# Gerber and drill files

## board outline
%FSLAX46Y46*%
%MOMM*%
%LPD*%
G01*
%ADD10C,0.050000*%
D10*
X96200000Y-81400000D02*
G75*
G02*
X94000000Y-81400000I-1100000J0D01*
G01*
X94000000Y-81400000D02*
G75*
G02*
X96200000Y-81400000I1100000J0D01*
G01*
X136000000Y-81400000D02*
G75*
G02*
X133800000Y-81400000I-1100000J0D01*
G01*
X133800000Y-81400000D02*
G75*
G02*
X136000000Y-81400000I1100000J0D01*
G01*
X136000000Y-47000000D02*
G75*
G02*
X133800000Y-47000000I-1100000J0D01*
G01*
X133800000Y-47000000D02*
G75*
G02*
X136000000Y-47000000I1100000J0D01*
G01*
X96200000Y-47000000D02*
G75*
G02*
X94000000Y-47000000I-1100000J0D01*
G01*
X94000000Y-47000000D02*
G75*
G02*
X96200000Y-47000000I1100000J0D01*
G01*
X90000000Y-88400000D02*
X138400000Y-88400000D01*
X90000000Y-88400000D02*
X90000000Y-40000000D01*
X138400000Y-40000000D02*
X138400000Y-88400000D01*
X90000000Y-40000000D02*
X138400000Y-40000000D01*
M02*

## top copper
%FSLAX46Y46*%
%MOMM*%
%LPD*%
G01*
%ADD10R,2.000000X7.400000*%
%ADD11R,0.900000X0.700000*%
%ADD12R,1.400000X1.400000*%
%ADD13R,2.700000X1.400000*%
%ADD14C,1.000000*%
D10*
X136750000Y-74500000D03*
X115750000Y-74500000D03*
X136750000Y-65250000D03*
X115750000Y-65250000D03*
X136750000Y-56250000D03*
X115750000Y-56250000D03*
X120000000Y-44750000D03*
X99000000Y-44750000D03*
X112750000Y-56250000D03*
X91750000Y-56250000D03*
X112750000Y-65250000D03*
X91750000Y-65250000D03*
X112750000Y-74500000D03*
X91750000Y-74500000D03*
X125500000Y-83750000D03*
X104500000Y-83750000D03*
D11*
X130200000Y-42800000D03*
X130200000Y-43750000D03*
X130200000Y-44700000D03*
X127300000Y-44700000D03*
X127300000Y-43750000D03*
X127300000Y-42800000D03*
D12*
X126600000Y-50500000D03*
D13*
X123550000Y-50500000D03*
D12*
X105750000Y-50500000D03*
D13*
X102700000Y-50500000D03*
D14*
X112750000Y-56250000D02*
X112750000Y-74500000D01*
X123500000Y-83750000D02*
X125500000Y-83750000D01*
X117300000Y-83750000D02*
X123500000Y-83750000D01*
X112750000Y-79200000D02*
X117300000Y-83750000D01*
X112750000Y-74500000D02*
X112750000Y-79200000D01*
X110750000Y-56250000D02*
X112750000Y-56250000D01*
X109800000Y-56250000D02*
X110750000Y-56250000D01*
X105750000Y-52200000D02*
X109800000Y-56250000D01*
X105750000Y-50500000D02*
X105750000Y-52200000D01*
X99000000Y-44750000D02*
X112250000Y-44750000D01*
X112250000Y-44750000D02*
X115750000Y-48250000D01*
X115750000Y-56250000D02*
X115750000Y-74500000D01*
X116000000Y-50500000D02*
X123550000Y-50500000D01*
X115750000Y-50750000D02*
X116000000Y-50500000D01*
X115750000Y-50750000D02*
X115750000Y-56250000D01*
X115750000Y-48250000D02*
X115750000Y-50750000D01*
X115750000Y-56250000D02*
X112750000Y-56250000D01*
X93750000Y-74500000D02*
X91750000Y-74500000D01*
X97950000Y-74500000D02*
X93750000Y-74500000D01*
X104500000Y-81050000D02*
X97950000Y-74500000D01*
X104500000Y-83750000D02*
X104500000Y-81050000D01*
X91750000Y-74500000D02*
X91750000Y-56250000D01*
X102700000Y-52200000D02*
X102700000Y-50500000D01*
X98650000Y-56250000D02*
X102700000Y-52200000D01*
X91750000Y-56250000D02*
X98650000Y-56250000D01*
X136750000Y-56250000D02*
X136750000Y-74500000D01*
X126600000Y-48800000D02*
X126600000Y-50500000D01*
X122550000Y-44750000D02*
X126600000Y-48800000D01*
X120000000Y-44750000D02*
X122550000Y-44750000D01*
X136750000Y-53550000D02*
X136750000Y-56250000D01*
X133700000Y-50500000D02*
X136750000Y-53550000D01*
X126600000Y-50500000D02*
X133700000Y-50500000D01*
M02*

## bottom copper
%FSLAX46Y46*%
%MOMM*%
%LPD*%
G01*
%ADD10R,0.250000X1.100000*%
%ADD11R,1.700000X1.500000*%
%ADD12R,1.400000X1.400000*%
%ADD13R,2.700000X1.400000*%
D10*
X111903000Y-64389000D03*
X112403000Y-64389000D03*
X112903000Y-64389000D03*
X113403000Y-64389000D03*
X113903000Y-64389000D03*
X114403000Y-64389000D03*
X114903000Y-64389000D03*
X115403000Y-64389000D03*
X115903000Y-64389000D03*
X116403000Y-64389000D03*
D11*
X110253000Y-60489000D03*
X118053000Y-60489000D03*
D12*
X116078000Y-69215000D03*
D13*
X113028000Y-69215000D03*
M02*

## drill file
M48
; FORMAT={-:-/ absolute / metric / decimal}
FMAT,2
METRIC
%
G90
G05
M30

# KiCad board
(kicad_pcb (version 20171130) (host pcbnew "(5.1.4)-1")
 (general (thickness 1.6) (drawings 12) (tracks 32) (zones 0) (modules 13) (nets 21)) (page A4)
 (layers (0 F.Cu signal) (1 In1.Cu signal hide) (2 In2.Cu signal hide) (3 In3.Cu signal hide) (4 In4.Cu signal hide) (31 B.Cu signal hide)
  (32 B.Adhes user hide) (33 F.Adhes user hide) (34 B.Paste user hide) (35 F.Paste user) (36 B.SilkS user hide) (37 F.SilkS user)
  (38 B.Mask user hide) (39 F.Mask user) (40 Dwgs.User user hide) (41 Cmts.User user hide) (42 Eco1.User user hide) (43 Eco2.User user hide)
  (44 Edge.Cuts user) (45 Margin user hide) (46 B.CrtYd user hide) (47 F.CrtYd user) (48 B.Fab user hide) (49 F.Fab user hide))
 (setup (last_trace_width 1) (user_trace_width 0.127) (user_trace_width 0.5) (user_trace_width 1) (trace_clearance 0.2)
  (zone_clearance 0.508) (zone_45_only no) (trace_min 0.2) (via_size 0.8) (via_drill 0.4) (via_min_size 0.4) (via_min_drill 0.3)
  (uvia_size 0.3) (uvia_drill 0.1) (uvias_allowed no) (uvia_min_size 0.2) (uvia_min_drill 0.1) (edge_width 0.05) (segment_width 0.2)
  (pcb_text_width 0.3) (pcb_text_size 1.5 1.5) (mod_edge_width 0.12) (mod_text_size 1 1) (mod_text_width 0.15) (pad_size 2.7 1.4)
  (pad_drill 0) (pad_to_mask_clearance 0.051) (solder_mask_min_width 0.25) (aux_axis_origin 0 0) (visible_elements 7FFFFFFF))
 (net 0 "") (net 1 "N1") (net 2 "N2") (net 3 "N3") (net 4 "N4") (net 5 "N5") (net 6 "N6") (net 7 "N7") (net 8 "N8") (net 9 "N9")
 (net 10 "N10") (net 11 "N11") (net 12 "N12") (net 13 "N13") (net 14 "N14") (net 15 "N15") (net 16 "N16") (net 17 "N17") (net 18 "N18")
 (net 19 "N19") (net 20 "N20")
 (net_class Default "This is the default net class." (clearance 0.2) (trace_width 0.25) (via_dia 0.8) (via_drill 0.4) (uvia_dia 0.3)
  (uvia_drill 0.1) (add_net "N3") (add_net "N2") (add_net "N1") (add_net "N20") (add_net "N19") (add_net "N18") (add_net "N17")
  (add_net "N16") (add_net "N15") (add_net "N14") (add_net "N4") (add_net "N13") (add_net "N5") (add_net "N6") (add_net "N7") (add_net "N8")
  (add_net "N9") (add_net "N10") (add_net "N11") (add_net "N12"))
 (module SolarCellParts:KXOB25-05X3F (layer F.Cu) (at 115.75 74.5)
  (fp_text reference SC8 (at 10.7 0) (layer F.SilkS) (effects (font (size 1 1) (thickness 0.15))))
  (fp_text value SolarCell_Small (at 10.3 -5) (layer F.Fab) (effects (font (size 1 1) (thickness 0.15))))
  (pad 2 smd rect (at 21 0) (size 2 7.4) (layers F.Cu F.Paste F.Mask) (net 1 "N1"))
  (pad 1 smd rect (at 0 0) (size 2 7.4) (layers F.Cu F.Paste F.Mask) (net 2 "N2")))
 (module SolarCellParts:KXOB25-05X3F (layer F.Cu) (at 115.75 65.25)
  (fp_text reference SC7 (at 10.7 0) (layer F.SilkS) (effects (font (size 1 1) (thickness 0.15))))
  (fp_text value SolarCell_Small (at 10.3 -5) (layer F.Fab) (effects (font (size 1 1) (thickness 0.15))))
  (pad 2 smd rect (at 21 0) (size 2 7.4) (layers F.Cu F.Paste F.Mask) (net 1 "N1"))
  (pad 1 smd rect (at 0 0) (size 2 7.4) (layers F.Cu F.Paste F.Mask) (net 2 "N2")))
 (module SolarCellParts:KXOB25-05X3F (layer F.Cu) (at 115.75 56.25)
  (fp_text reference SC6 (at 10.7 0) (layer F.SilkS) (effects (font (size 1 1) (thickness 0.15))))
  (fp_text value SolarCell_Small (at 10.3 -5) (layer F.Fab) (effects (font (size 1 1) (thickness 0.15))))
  (pad 2 smd rect (at 21 0) (size 2 7.4) (layers F.Cu F.Paste F.Mask) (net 1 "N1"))
  (pad 1 smd rect (at 0 0) (size 2 7.4) (layers F.Cu F.Paste F.Mask) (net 2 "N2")))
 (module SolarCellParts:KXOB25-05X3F (layer F.Cu) (at 99 44.75)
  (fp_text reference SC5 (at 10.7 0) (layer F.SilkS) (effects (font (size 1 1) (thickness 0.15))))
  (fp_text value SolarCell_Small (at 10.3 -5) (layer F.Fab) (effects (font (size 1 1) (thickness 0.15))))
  (pad 2 smd rect (at 21 0) (size 2 7.4) (layers F.Cu F.Paste F.Mask) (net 1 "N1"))
  (pad 1 smd rect (at 0 0) (size 2 7.4) (layers F.Cu F.Paste F.Mask) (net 2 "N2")))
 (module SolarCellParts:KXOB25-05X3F (layer F.Cu) (at 91.75 56.25)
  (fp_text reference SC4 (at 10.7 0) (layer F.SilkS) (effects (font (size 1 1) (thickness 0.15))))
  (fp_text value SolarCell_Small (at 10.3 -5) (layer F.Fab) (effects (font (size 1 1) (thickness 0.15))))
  (pad 2 smd rect (at 21 0) (size 2 7.4) (layers F.Cu F.Paste F.Mask) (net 2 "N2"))
  (pad 1 smd rect (at 0 0) (size 2 7.4) (layers F.Cu F.Paste F.Mask) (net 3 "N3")))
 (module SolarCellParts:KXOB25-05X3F (layer F.Cu) (at 91.75 65.25)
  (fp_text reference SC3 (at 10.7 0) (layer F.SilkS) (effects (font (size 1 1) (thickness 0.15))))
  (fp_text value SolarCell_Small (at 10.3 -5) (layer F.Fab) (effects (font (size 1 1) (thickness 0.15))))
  (pad 2 smd rect (at 21 0) (size 2 7.4) (layers F.Cu F.Paste F.Mask) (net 2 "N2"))
  (pad 1 smd rect (at 0 0) (size 2 7.4) (layers F.Cu F.Paste F.Mask) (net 3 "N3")))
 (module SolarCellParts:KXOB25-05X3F (layer F.Cu) (at 91.75 74.5)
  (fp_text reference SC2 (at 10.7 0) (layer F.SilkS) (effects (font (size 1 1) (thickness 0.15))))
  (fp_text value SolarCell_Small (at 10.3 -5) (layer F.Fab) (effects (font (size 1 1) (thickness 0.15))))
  (pad 2 smd rect (at 21 0) (size 2 7.4) (layers F.Cu F.Paste F.Mask) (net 2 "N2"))
  (pad 1 smd rect (at 0 0) (size 2 7.4) (layers F.Cu F.Paste F.Mask) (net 3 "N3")))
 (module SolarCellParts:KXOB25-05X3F (layer F.Cu) (at 104.5 83.75)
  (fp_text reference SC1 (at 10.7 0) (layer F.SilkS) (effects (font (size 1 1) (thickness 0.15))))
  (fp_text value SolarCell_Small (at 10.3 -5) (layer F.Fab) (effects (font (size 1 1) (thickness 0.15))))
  (pad 2 smd rect (at 21 0) (size 2 7.4) (layers F.Cu F.Paste F.Mask) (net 2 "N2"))
  (pad 1 smd rect (at 0 0) (size 2 7.4) (layers F.Cu F.Paste F.Mask) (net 3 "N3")))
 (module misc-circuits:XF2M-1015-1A (layer B.Cu) (at 114.153 64.389)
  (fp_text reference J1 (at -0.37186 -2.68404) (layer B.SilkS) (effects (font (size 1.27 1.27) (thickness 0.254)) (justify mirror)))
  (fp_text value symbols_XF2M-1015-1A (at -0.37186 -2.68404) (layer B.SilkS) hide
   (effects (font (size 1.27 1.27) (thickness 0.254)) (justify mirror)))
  (pad 1 smd rect (at -2.25 0) (size 0.25 1.1) (layers B.Cu B.Paste B.Mask) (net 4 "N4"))
  (pad 2 smd rect (at -1.75 0) (size 0.25 1.1) (layers B.Cu B.Paste B.Mask) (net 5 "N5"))
  (pad 3 smd rect (at -1.25 0) (size 0.25 1.1) (layers B.Cu B.Paste B.Mask) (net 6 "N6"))
  (pad 4 smd rect (at -0.75 0) (size 0.25 1.1) (layers B.Cu B.Paste B.Mask) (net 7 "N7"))
  (pad 5 smd rect (at -0.25 0) (size 0.25 1.1) (layers B.Cu B.Paste B.Mask) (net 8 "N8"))
  (pad 6 smd rect (at 0.25 0) (size 0.25 1.1) (layers B.Cu B.Paste B.Mask) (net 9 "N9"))
  (pad 7 smd rect (at 0.75 0) (size 0.25 1.1) (layers B.Cu B.Paste B.Mask) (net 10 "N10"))
  (pad 8 smd rect (at 1.25 0) (size 0.25 1.1) (layers B.Cu B.Paste B.Mask) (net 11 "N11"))
  (pad 9 smd rect (at 1.75 0) (size 0.25 1.1) (layers B.Cu B.Paste B.Mask) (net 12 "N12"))
  (pad 10 smd rect (at 2.25 0) (size 0.25 1.1) (layers B.Cu B.Paste B.Mask) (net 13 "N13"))
  (pad 11 smd rect (at -3.9 -3.9 270) (size 1.5 1.7) (layers B.Cu B.Paste B.Mask))
  (pad 12 smd rect (at 3.9 -3.9 270) (size 1.5 1.7) (layers B.Cu B.Paste B.Mask)))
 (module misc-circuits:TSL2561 (layer F.Cu) (at 128.75 43.75)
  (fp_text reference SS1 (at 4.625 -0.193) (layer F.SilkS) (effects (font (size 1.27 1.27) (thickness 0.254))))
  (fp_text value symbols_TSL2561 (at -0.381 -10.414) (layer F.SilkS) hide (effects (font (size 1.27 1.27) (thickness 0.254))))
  (pad 6 smd rect (at 1.45 -0.95 90) (size 0.7 0.9) (layers F.Cu F.Paste F.Mask) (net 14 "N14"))
  (pad 5 smd rect (at 1.45 0 90) (size 0.7 0.9) (layers F.Cu F.Paste F.Mask) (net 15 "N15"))
  (pad 4 smd rect (at 1.45 0.95 90) (size 0.7 0.9) (layers F.Cu F.Paste F.Mask) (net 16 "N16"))
  (pad 3 smd rect (at -1.45 0.95 90) (size 0.7 0.9) (layers F.Cu F.Paste F.Mask) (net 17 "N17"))
  (pad 2 smd rect (at -1.45 0 90) (size 0.7 0.9) (layers F.Cu F.Paste F.Mask) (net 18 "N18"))
  (pad 1 smd rect (at -1.45 -0.95 90) (size 0.7 0.9) (layers F.Cu F.Paste F.Mask) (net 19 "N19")))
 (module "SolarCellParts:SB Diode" (layer B.Cu) (at 114.228 69.215)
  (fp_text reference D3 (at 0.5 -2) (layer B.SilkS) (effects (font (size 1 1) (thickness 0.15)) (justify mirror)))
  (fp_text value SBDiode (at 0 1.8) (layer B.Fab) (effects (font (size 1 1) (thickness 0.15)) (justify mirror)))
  (pad 2 smd rect (at 1.85 0) (size 1.4 1.4) (layers B.Cu B.Paste B.Mask) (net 3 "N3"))
  (pad 1 smd rect (at -1.2 0) (size 2.7 1.4) (layers B.Cu B.Paste B.Mask) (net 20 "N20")))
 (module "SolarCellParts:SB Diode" (layer F.Cu) (at 124.75 50.5)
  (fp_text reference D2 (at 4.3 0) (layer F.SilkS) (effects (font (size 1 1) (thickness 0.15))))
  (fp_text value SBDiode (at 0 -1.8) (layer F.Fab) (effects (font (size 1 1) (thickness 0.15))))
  (pad 2 smd rect (at 1.85 0) (size 1.4 1.4) (layers F.Cu F.Paste F.Mask) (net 1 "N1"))
  (pad 1 smd rect (at -1.2 0) (size 2.7 1.4) (layers F.Cu F.Paste F.Mask) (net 2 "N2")))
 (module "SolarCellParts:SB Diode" (layer F.Cu) (at 103.9 50.5)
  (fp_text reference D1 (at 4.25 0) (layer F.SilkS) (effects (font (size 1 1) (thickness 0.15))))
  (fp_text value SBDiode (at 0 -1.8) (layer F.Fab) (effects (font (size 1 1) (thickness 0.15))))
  (pad 2 smd rect (at 1.85 0) (size 1.4 1.4) (layers F.Cu F.Paste F.Mask) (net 2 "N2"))
  (pad 1 smd rect (at -1.2 0) (size 2.7 1.4) (layers F.Cu F.Paste F.Mask) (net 3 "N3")))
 (gr_circle (center 95.1 81.4) (end 96.2 81.4) (layer Edge.Cuts) (width 0.05))
 (gr_circle (center 134.9 81.4) (end 136 81.4) (layer Edge.Cuts) (width 0.05))
 (gr_circle (center 134.9 47) (end 136 47) (layer Edge.Cuts) (width 0.05))
 (gr_circle (center 95.1 47) (end 96.2 47) (layer Edge.Cuts) (width 0.05))
 (gr_line (start 90 88.4) (end 138.4 88.4) (layer Edge.Cuts) (width 0.05))
 (gr_line (start 90 88.4) (end 90 40) (layer Edge.Cuts) (width 0.05))
 (gr_line (start 138.4 40) (end 138.4 88.4) (layer Edge.Cuts) (width 0.05))
 (gr_line (start 90 40) (end 138.4 40) (layer Edge.Cuts) (width 0.05))
 (segment (start 112.75 56.25) (end 112.75 74.5) (width 1) (layer F.Cu) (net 2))
 (segment (start 123.5 83.75) (end 125.5 83.75) (width 1) (layer F.Cu) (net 2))
 (segment (start 117.3 83.75) (end 123.5 83.75) (width 1) (layer F.Cu) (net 2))
 (segment (start 112.75 79.2) (end 117.3 83.75) (width 1) (layer F.Cu) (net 2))
 (segment (start 112.75 74.5) (end 112.75 79.2) (width 1) (layer F.Cu) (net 2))
 (segment (start 110.75 56.25) (end 112.75 56.25) (width 1) (layer F.Cu) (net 2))
 (segment (start 109.8 56.25) (end 110.75 56.25) (width 1) (layer F.Cu) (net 2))
 (segment (start 105.75 52.2) (end 109.8 56.25) (width 1) (layer F.Cu) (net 2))
 (segment (start 105.75 50.5) (end 105.75 52.2) (width 1) (layer F.Cu) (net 2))
 (segment (start 99 44.75) (end 112.25 44.75) (width 1) (layer F.Cu) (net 2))
 (segment (start 112.25 44.75) (end 115.75 48.25) (width 1) (layer F.Cu) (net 2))
 (segment (start 115.75 56.25) (end 115.75 74.5) (width 1) (layer F.Cu) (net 2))
 (segment (start 116 50.5) (end 123.55 50.5) (width 1) (layer F.Cu) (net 2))
 (segment (start 115.75 50.75) (end 116 50.5) (width 1) (layer F.Cu) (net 2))
 (segment (start 115.75 50.75) (end 115.75 56.25) (width 1) (layer F.Cu) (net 2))
 (segment (start 115.75 48.25) (end 115.75 50.75) (width 1) (layer F.Cu) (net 2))
 (segment (start 115.75 56.25) (end 112.75 56.25) (width 1) (layer F.Cu) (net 2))
 (segment (start 93.75 74.5) (end 91.75 74.5) (width 1) (layer F.Cu) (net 3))
 (segment (start 97.95 74.5) (end 93.75 74.5) (width 1) (layer F.Cu) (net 3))
 (segment (start 104.5 81.05) (end 97.95 74.5) (width 1) (layer F.Cu) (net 3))
 (segment (start 104.5 83.75) (end 104.5 81.05) (width 1) (layer F.Cu) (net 3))
 (segment (start 91.75 74.5) (end 91.75 56.25) (width 1) (layer F.Cu) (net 3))
 (segment (start 102.7 52.2) (end 102.7 50.5) (width 1) (layer F.Cu) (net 3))
 (segment (start 98.65 56.25) (end 102.7 52.2) (width 1) (layer F.Cu) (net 3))
 (segment (start 91.75 56.25) (end 98.65 56.25) (width 1) (layer F.Cu) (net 3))
 (segment (start 136.75 56.25) (end 136.75 74.5) (width 1) (layer F.Cu) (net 1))
 (segment (start 126.6 48.8) (end 126.6 50.5) (width 1) (layer F.Cu) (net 1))
 (segment (start 122.55 44.75) (end 126.6 48.8) (width 1) (layer F.Cu) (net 1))
 (segment (start 120 44.75) (end 122.55 44.75) (width 1) (layer F.Cu) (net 1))
 (segment (start 136.75 53.55) (end 136.75 56.25) (width 1) (layer F.Cu) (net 1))
 (segment (start 133.7 50.5) (end 136.75 53.55) (width 1) (layer F.Cu) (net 1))
 (segment (start 126.6 50.5) (end 133.7 50.5) (width 1) (layer F.Cu) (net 1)))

